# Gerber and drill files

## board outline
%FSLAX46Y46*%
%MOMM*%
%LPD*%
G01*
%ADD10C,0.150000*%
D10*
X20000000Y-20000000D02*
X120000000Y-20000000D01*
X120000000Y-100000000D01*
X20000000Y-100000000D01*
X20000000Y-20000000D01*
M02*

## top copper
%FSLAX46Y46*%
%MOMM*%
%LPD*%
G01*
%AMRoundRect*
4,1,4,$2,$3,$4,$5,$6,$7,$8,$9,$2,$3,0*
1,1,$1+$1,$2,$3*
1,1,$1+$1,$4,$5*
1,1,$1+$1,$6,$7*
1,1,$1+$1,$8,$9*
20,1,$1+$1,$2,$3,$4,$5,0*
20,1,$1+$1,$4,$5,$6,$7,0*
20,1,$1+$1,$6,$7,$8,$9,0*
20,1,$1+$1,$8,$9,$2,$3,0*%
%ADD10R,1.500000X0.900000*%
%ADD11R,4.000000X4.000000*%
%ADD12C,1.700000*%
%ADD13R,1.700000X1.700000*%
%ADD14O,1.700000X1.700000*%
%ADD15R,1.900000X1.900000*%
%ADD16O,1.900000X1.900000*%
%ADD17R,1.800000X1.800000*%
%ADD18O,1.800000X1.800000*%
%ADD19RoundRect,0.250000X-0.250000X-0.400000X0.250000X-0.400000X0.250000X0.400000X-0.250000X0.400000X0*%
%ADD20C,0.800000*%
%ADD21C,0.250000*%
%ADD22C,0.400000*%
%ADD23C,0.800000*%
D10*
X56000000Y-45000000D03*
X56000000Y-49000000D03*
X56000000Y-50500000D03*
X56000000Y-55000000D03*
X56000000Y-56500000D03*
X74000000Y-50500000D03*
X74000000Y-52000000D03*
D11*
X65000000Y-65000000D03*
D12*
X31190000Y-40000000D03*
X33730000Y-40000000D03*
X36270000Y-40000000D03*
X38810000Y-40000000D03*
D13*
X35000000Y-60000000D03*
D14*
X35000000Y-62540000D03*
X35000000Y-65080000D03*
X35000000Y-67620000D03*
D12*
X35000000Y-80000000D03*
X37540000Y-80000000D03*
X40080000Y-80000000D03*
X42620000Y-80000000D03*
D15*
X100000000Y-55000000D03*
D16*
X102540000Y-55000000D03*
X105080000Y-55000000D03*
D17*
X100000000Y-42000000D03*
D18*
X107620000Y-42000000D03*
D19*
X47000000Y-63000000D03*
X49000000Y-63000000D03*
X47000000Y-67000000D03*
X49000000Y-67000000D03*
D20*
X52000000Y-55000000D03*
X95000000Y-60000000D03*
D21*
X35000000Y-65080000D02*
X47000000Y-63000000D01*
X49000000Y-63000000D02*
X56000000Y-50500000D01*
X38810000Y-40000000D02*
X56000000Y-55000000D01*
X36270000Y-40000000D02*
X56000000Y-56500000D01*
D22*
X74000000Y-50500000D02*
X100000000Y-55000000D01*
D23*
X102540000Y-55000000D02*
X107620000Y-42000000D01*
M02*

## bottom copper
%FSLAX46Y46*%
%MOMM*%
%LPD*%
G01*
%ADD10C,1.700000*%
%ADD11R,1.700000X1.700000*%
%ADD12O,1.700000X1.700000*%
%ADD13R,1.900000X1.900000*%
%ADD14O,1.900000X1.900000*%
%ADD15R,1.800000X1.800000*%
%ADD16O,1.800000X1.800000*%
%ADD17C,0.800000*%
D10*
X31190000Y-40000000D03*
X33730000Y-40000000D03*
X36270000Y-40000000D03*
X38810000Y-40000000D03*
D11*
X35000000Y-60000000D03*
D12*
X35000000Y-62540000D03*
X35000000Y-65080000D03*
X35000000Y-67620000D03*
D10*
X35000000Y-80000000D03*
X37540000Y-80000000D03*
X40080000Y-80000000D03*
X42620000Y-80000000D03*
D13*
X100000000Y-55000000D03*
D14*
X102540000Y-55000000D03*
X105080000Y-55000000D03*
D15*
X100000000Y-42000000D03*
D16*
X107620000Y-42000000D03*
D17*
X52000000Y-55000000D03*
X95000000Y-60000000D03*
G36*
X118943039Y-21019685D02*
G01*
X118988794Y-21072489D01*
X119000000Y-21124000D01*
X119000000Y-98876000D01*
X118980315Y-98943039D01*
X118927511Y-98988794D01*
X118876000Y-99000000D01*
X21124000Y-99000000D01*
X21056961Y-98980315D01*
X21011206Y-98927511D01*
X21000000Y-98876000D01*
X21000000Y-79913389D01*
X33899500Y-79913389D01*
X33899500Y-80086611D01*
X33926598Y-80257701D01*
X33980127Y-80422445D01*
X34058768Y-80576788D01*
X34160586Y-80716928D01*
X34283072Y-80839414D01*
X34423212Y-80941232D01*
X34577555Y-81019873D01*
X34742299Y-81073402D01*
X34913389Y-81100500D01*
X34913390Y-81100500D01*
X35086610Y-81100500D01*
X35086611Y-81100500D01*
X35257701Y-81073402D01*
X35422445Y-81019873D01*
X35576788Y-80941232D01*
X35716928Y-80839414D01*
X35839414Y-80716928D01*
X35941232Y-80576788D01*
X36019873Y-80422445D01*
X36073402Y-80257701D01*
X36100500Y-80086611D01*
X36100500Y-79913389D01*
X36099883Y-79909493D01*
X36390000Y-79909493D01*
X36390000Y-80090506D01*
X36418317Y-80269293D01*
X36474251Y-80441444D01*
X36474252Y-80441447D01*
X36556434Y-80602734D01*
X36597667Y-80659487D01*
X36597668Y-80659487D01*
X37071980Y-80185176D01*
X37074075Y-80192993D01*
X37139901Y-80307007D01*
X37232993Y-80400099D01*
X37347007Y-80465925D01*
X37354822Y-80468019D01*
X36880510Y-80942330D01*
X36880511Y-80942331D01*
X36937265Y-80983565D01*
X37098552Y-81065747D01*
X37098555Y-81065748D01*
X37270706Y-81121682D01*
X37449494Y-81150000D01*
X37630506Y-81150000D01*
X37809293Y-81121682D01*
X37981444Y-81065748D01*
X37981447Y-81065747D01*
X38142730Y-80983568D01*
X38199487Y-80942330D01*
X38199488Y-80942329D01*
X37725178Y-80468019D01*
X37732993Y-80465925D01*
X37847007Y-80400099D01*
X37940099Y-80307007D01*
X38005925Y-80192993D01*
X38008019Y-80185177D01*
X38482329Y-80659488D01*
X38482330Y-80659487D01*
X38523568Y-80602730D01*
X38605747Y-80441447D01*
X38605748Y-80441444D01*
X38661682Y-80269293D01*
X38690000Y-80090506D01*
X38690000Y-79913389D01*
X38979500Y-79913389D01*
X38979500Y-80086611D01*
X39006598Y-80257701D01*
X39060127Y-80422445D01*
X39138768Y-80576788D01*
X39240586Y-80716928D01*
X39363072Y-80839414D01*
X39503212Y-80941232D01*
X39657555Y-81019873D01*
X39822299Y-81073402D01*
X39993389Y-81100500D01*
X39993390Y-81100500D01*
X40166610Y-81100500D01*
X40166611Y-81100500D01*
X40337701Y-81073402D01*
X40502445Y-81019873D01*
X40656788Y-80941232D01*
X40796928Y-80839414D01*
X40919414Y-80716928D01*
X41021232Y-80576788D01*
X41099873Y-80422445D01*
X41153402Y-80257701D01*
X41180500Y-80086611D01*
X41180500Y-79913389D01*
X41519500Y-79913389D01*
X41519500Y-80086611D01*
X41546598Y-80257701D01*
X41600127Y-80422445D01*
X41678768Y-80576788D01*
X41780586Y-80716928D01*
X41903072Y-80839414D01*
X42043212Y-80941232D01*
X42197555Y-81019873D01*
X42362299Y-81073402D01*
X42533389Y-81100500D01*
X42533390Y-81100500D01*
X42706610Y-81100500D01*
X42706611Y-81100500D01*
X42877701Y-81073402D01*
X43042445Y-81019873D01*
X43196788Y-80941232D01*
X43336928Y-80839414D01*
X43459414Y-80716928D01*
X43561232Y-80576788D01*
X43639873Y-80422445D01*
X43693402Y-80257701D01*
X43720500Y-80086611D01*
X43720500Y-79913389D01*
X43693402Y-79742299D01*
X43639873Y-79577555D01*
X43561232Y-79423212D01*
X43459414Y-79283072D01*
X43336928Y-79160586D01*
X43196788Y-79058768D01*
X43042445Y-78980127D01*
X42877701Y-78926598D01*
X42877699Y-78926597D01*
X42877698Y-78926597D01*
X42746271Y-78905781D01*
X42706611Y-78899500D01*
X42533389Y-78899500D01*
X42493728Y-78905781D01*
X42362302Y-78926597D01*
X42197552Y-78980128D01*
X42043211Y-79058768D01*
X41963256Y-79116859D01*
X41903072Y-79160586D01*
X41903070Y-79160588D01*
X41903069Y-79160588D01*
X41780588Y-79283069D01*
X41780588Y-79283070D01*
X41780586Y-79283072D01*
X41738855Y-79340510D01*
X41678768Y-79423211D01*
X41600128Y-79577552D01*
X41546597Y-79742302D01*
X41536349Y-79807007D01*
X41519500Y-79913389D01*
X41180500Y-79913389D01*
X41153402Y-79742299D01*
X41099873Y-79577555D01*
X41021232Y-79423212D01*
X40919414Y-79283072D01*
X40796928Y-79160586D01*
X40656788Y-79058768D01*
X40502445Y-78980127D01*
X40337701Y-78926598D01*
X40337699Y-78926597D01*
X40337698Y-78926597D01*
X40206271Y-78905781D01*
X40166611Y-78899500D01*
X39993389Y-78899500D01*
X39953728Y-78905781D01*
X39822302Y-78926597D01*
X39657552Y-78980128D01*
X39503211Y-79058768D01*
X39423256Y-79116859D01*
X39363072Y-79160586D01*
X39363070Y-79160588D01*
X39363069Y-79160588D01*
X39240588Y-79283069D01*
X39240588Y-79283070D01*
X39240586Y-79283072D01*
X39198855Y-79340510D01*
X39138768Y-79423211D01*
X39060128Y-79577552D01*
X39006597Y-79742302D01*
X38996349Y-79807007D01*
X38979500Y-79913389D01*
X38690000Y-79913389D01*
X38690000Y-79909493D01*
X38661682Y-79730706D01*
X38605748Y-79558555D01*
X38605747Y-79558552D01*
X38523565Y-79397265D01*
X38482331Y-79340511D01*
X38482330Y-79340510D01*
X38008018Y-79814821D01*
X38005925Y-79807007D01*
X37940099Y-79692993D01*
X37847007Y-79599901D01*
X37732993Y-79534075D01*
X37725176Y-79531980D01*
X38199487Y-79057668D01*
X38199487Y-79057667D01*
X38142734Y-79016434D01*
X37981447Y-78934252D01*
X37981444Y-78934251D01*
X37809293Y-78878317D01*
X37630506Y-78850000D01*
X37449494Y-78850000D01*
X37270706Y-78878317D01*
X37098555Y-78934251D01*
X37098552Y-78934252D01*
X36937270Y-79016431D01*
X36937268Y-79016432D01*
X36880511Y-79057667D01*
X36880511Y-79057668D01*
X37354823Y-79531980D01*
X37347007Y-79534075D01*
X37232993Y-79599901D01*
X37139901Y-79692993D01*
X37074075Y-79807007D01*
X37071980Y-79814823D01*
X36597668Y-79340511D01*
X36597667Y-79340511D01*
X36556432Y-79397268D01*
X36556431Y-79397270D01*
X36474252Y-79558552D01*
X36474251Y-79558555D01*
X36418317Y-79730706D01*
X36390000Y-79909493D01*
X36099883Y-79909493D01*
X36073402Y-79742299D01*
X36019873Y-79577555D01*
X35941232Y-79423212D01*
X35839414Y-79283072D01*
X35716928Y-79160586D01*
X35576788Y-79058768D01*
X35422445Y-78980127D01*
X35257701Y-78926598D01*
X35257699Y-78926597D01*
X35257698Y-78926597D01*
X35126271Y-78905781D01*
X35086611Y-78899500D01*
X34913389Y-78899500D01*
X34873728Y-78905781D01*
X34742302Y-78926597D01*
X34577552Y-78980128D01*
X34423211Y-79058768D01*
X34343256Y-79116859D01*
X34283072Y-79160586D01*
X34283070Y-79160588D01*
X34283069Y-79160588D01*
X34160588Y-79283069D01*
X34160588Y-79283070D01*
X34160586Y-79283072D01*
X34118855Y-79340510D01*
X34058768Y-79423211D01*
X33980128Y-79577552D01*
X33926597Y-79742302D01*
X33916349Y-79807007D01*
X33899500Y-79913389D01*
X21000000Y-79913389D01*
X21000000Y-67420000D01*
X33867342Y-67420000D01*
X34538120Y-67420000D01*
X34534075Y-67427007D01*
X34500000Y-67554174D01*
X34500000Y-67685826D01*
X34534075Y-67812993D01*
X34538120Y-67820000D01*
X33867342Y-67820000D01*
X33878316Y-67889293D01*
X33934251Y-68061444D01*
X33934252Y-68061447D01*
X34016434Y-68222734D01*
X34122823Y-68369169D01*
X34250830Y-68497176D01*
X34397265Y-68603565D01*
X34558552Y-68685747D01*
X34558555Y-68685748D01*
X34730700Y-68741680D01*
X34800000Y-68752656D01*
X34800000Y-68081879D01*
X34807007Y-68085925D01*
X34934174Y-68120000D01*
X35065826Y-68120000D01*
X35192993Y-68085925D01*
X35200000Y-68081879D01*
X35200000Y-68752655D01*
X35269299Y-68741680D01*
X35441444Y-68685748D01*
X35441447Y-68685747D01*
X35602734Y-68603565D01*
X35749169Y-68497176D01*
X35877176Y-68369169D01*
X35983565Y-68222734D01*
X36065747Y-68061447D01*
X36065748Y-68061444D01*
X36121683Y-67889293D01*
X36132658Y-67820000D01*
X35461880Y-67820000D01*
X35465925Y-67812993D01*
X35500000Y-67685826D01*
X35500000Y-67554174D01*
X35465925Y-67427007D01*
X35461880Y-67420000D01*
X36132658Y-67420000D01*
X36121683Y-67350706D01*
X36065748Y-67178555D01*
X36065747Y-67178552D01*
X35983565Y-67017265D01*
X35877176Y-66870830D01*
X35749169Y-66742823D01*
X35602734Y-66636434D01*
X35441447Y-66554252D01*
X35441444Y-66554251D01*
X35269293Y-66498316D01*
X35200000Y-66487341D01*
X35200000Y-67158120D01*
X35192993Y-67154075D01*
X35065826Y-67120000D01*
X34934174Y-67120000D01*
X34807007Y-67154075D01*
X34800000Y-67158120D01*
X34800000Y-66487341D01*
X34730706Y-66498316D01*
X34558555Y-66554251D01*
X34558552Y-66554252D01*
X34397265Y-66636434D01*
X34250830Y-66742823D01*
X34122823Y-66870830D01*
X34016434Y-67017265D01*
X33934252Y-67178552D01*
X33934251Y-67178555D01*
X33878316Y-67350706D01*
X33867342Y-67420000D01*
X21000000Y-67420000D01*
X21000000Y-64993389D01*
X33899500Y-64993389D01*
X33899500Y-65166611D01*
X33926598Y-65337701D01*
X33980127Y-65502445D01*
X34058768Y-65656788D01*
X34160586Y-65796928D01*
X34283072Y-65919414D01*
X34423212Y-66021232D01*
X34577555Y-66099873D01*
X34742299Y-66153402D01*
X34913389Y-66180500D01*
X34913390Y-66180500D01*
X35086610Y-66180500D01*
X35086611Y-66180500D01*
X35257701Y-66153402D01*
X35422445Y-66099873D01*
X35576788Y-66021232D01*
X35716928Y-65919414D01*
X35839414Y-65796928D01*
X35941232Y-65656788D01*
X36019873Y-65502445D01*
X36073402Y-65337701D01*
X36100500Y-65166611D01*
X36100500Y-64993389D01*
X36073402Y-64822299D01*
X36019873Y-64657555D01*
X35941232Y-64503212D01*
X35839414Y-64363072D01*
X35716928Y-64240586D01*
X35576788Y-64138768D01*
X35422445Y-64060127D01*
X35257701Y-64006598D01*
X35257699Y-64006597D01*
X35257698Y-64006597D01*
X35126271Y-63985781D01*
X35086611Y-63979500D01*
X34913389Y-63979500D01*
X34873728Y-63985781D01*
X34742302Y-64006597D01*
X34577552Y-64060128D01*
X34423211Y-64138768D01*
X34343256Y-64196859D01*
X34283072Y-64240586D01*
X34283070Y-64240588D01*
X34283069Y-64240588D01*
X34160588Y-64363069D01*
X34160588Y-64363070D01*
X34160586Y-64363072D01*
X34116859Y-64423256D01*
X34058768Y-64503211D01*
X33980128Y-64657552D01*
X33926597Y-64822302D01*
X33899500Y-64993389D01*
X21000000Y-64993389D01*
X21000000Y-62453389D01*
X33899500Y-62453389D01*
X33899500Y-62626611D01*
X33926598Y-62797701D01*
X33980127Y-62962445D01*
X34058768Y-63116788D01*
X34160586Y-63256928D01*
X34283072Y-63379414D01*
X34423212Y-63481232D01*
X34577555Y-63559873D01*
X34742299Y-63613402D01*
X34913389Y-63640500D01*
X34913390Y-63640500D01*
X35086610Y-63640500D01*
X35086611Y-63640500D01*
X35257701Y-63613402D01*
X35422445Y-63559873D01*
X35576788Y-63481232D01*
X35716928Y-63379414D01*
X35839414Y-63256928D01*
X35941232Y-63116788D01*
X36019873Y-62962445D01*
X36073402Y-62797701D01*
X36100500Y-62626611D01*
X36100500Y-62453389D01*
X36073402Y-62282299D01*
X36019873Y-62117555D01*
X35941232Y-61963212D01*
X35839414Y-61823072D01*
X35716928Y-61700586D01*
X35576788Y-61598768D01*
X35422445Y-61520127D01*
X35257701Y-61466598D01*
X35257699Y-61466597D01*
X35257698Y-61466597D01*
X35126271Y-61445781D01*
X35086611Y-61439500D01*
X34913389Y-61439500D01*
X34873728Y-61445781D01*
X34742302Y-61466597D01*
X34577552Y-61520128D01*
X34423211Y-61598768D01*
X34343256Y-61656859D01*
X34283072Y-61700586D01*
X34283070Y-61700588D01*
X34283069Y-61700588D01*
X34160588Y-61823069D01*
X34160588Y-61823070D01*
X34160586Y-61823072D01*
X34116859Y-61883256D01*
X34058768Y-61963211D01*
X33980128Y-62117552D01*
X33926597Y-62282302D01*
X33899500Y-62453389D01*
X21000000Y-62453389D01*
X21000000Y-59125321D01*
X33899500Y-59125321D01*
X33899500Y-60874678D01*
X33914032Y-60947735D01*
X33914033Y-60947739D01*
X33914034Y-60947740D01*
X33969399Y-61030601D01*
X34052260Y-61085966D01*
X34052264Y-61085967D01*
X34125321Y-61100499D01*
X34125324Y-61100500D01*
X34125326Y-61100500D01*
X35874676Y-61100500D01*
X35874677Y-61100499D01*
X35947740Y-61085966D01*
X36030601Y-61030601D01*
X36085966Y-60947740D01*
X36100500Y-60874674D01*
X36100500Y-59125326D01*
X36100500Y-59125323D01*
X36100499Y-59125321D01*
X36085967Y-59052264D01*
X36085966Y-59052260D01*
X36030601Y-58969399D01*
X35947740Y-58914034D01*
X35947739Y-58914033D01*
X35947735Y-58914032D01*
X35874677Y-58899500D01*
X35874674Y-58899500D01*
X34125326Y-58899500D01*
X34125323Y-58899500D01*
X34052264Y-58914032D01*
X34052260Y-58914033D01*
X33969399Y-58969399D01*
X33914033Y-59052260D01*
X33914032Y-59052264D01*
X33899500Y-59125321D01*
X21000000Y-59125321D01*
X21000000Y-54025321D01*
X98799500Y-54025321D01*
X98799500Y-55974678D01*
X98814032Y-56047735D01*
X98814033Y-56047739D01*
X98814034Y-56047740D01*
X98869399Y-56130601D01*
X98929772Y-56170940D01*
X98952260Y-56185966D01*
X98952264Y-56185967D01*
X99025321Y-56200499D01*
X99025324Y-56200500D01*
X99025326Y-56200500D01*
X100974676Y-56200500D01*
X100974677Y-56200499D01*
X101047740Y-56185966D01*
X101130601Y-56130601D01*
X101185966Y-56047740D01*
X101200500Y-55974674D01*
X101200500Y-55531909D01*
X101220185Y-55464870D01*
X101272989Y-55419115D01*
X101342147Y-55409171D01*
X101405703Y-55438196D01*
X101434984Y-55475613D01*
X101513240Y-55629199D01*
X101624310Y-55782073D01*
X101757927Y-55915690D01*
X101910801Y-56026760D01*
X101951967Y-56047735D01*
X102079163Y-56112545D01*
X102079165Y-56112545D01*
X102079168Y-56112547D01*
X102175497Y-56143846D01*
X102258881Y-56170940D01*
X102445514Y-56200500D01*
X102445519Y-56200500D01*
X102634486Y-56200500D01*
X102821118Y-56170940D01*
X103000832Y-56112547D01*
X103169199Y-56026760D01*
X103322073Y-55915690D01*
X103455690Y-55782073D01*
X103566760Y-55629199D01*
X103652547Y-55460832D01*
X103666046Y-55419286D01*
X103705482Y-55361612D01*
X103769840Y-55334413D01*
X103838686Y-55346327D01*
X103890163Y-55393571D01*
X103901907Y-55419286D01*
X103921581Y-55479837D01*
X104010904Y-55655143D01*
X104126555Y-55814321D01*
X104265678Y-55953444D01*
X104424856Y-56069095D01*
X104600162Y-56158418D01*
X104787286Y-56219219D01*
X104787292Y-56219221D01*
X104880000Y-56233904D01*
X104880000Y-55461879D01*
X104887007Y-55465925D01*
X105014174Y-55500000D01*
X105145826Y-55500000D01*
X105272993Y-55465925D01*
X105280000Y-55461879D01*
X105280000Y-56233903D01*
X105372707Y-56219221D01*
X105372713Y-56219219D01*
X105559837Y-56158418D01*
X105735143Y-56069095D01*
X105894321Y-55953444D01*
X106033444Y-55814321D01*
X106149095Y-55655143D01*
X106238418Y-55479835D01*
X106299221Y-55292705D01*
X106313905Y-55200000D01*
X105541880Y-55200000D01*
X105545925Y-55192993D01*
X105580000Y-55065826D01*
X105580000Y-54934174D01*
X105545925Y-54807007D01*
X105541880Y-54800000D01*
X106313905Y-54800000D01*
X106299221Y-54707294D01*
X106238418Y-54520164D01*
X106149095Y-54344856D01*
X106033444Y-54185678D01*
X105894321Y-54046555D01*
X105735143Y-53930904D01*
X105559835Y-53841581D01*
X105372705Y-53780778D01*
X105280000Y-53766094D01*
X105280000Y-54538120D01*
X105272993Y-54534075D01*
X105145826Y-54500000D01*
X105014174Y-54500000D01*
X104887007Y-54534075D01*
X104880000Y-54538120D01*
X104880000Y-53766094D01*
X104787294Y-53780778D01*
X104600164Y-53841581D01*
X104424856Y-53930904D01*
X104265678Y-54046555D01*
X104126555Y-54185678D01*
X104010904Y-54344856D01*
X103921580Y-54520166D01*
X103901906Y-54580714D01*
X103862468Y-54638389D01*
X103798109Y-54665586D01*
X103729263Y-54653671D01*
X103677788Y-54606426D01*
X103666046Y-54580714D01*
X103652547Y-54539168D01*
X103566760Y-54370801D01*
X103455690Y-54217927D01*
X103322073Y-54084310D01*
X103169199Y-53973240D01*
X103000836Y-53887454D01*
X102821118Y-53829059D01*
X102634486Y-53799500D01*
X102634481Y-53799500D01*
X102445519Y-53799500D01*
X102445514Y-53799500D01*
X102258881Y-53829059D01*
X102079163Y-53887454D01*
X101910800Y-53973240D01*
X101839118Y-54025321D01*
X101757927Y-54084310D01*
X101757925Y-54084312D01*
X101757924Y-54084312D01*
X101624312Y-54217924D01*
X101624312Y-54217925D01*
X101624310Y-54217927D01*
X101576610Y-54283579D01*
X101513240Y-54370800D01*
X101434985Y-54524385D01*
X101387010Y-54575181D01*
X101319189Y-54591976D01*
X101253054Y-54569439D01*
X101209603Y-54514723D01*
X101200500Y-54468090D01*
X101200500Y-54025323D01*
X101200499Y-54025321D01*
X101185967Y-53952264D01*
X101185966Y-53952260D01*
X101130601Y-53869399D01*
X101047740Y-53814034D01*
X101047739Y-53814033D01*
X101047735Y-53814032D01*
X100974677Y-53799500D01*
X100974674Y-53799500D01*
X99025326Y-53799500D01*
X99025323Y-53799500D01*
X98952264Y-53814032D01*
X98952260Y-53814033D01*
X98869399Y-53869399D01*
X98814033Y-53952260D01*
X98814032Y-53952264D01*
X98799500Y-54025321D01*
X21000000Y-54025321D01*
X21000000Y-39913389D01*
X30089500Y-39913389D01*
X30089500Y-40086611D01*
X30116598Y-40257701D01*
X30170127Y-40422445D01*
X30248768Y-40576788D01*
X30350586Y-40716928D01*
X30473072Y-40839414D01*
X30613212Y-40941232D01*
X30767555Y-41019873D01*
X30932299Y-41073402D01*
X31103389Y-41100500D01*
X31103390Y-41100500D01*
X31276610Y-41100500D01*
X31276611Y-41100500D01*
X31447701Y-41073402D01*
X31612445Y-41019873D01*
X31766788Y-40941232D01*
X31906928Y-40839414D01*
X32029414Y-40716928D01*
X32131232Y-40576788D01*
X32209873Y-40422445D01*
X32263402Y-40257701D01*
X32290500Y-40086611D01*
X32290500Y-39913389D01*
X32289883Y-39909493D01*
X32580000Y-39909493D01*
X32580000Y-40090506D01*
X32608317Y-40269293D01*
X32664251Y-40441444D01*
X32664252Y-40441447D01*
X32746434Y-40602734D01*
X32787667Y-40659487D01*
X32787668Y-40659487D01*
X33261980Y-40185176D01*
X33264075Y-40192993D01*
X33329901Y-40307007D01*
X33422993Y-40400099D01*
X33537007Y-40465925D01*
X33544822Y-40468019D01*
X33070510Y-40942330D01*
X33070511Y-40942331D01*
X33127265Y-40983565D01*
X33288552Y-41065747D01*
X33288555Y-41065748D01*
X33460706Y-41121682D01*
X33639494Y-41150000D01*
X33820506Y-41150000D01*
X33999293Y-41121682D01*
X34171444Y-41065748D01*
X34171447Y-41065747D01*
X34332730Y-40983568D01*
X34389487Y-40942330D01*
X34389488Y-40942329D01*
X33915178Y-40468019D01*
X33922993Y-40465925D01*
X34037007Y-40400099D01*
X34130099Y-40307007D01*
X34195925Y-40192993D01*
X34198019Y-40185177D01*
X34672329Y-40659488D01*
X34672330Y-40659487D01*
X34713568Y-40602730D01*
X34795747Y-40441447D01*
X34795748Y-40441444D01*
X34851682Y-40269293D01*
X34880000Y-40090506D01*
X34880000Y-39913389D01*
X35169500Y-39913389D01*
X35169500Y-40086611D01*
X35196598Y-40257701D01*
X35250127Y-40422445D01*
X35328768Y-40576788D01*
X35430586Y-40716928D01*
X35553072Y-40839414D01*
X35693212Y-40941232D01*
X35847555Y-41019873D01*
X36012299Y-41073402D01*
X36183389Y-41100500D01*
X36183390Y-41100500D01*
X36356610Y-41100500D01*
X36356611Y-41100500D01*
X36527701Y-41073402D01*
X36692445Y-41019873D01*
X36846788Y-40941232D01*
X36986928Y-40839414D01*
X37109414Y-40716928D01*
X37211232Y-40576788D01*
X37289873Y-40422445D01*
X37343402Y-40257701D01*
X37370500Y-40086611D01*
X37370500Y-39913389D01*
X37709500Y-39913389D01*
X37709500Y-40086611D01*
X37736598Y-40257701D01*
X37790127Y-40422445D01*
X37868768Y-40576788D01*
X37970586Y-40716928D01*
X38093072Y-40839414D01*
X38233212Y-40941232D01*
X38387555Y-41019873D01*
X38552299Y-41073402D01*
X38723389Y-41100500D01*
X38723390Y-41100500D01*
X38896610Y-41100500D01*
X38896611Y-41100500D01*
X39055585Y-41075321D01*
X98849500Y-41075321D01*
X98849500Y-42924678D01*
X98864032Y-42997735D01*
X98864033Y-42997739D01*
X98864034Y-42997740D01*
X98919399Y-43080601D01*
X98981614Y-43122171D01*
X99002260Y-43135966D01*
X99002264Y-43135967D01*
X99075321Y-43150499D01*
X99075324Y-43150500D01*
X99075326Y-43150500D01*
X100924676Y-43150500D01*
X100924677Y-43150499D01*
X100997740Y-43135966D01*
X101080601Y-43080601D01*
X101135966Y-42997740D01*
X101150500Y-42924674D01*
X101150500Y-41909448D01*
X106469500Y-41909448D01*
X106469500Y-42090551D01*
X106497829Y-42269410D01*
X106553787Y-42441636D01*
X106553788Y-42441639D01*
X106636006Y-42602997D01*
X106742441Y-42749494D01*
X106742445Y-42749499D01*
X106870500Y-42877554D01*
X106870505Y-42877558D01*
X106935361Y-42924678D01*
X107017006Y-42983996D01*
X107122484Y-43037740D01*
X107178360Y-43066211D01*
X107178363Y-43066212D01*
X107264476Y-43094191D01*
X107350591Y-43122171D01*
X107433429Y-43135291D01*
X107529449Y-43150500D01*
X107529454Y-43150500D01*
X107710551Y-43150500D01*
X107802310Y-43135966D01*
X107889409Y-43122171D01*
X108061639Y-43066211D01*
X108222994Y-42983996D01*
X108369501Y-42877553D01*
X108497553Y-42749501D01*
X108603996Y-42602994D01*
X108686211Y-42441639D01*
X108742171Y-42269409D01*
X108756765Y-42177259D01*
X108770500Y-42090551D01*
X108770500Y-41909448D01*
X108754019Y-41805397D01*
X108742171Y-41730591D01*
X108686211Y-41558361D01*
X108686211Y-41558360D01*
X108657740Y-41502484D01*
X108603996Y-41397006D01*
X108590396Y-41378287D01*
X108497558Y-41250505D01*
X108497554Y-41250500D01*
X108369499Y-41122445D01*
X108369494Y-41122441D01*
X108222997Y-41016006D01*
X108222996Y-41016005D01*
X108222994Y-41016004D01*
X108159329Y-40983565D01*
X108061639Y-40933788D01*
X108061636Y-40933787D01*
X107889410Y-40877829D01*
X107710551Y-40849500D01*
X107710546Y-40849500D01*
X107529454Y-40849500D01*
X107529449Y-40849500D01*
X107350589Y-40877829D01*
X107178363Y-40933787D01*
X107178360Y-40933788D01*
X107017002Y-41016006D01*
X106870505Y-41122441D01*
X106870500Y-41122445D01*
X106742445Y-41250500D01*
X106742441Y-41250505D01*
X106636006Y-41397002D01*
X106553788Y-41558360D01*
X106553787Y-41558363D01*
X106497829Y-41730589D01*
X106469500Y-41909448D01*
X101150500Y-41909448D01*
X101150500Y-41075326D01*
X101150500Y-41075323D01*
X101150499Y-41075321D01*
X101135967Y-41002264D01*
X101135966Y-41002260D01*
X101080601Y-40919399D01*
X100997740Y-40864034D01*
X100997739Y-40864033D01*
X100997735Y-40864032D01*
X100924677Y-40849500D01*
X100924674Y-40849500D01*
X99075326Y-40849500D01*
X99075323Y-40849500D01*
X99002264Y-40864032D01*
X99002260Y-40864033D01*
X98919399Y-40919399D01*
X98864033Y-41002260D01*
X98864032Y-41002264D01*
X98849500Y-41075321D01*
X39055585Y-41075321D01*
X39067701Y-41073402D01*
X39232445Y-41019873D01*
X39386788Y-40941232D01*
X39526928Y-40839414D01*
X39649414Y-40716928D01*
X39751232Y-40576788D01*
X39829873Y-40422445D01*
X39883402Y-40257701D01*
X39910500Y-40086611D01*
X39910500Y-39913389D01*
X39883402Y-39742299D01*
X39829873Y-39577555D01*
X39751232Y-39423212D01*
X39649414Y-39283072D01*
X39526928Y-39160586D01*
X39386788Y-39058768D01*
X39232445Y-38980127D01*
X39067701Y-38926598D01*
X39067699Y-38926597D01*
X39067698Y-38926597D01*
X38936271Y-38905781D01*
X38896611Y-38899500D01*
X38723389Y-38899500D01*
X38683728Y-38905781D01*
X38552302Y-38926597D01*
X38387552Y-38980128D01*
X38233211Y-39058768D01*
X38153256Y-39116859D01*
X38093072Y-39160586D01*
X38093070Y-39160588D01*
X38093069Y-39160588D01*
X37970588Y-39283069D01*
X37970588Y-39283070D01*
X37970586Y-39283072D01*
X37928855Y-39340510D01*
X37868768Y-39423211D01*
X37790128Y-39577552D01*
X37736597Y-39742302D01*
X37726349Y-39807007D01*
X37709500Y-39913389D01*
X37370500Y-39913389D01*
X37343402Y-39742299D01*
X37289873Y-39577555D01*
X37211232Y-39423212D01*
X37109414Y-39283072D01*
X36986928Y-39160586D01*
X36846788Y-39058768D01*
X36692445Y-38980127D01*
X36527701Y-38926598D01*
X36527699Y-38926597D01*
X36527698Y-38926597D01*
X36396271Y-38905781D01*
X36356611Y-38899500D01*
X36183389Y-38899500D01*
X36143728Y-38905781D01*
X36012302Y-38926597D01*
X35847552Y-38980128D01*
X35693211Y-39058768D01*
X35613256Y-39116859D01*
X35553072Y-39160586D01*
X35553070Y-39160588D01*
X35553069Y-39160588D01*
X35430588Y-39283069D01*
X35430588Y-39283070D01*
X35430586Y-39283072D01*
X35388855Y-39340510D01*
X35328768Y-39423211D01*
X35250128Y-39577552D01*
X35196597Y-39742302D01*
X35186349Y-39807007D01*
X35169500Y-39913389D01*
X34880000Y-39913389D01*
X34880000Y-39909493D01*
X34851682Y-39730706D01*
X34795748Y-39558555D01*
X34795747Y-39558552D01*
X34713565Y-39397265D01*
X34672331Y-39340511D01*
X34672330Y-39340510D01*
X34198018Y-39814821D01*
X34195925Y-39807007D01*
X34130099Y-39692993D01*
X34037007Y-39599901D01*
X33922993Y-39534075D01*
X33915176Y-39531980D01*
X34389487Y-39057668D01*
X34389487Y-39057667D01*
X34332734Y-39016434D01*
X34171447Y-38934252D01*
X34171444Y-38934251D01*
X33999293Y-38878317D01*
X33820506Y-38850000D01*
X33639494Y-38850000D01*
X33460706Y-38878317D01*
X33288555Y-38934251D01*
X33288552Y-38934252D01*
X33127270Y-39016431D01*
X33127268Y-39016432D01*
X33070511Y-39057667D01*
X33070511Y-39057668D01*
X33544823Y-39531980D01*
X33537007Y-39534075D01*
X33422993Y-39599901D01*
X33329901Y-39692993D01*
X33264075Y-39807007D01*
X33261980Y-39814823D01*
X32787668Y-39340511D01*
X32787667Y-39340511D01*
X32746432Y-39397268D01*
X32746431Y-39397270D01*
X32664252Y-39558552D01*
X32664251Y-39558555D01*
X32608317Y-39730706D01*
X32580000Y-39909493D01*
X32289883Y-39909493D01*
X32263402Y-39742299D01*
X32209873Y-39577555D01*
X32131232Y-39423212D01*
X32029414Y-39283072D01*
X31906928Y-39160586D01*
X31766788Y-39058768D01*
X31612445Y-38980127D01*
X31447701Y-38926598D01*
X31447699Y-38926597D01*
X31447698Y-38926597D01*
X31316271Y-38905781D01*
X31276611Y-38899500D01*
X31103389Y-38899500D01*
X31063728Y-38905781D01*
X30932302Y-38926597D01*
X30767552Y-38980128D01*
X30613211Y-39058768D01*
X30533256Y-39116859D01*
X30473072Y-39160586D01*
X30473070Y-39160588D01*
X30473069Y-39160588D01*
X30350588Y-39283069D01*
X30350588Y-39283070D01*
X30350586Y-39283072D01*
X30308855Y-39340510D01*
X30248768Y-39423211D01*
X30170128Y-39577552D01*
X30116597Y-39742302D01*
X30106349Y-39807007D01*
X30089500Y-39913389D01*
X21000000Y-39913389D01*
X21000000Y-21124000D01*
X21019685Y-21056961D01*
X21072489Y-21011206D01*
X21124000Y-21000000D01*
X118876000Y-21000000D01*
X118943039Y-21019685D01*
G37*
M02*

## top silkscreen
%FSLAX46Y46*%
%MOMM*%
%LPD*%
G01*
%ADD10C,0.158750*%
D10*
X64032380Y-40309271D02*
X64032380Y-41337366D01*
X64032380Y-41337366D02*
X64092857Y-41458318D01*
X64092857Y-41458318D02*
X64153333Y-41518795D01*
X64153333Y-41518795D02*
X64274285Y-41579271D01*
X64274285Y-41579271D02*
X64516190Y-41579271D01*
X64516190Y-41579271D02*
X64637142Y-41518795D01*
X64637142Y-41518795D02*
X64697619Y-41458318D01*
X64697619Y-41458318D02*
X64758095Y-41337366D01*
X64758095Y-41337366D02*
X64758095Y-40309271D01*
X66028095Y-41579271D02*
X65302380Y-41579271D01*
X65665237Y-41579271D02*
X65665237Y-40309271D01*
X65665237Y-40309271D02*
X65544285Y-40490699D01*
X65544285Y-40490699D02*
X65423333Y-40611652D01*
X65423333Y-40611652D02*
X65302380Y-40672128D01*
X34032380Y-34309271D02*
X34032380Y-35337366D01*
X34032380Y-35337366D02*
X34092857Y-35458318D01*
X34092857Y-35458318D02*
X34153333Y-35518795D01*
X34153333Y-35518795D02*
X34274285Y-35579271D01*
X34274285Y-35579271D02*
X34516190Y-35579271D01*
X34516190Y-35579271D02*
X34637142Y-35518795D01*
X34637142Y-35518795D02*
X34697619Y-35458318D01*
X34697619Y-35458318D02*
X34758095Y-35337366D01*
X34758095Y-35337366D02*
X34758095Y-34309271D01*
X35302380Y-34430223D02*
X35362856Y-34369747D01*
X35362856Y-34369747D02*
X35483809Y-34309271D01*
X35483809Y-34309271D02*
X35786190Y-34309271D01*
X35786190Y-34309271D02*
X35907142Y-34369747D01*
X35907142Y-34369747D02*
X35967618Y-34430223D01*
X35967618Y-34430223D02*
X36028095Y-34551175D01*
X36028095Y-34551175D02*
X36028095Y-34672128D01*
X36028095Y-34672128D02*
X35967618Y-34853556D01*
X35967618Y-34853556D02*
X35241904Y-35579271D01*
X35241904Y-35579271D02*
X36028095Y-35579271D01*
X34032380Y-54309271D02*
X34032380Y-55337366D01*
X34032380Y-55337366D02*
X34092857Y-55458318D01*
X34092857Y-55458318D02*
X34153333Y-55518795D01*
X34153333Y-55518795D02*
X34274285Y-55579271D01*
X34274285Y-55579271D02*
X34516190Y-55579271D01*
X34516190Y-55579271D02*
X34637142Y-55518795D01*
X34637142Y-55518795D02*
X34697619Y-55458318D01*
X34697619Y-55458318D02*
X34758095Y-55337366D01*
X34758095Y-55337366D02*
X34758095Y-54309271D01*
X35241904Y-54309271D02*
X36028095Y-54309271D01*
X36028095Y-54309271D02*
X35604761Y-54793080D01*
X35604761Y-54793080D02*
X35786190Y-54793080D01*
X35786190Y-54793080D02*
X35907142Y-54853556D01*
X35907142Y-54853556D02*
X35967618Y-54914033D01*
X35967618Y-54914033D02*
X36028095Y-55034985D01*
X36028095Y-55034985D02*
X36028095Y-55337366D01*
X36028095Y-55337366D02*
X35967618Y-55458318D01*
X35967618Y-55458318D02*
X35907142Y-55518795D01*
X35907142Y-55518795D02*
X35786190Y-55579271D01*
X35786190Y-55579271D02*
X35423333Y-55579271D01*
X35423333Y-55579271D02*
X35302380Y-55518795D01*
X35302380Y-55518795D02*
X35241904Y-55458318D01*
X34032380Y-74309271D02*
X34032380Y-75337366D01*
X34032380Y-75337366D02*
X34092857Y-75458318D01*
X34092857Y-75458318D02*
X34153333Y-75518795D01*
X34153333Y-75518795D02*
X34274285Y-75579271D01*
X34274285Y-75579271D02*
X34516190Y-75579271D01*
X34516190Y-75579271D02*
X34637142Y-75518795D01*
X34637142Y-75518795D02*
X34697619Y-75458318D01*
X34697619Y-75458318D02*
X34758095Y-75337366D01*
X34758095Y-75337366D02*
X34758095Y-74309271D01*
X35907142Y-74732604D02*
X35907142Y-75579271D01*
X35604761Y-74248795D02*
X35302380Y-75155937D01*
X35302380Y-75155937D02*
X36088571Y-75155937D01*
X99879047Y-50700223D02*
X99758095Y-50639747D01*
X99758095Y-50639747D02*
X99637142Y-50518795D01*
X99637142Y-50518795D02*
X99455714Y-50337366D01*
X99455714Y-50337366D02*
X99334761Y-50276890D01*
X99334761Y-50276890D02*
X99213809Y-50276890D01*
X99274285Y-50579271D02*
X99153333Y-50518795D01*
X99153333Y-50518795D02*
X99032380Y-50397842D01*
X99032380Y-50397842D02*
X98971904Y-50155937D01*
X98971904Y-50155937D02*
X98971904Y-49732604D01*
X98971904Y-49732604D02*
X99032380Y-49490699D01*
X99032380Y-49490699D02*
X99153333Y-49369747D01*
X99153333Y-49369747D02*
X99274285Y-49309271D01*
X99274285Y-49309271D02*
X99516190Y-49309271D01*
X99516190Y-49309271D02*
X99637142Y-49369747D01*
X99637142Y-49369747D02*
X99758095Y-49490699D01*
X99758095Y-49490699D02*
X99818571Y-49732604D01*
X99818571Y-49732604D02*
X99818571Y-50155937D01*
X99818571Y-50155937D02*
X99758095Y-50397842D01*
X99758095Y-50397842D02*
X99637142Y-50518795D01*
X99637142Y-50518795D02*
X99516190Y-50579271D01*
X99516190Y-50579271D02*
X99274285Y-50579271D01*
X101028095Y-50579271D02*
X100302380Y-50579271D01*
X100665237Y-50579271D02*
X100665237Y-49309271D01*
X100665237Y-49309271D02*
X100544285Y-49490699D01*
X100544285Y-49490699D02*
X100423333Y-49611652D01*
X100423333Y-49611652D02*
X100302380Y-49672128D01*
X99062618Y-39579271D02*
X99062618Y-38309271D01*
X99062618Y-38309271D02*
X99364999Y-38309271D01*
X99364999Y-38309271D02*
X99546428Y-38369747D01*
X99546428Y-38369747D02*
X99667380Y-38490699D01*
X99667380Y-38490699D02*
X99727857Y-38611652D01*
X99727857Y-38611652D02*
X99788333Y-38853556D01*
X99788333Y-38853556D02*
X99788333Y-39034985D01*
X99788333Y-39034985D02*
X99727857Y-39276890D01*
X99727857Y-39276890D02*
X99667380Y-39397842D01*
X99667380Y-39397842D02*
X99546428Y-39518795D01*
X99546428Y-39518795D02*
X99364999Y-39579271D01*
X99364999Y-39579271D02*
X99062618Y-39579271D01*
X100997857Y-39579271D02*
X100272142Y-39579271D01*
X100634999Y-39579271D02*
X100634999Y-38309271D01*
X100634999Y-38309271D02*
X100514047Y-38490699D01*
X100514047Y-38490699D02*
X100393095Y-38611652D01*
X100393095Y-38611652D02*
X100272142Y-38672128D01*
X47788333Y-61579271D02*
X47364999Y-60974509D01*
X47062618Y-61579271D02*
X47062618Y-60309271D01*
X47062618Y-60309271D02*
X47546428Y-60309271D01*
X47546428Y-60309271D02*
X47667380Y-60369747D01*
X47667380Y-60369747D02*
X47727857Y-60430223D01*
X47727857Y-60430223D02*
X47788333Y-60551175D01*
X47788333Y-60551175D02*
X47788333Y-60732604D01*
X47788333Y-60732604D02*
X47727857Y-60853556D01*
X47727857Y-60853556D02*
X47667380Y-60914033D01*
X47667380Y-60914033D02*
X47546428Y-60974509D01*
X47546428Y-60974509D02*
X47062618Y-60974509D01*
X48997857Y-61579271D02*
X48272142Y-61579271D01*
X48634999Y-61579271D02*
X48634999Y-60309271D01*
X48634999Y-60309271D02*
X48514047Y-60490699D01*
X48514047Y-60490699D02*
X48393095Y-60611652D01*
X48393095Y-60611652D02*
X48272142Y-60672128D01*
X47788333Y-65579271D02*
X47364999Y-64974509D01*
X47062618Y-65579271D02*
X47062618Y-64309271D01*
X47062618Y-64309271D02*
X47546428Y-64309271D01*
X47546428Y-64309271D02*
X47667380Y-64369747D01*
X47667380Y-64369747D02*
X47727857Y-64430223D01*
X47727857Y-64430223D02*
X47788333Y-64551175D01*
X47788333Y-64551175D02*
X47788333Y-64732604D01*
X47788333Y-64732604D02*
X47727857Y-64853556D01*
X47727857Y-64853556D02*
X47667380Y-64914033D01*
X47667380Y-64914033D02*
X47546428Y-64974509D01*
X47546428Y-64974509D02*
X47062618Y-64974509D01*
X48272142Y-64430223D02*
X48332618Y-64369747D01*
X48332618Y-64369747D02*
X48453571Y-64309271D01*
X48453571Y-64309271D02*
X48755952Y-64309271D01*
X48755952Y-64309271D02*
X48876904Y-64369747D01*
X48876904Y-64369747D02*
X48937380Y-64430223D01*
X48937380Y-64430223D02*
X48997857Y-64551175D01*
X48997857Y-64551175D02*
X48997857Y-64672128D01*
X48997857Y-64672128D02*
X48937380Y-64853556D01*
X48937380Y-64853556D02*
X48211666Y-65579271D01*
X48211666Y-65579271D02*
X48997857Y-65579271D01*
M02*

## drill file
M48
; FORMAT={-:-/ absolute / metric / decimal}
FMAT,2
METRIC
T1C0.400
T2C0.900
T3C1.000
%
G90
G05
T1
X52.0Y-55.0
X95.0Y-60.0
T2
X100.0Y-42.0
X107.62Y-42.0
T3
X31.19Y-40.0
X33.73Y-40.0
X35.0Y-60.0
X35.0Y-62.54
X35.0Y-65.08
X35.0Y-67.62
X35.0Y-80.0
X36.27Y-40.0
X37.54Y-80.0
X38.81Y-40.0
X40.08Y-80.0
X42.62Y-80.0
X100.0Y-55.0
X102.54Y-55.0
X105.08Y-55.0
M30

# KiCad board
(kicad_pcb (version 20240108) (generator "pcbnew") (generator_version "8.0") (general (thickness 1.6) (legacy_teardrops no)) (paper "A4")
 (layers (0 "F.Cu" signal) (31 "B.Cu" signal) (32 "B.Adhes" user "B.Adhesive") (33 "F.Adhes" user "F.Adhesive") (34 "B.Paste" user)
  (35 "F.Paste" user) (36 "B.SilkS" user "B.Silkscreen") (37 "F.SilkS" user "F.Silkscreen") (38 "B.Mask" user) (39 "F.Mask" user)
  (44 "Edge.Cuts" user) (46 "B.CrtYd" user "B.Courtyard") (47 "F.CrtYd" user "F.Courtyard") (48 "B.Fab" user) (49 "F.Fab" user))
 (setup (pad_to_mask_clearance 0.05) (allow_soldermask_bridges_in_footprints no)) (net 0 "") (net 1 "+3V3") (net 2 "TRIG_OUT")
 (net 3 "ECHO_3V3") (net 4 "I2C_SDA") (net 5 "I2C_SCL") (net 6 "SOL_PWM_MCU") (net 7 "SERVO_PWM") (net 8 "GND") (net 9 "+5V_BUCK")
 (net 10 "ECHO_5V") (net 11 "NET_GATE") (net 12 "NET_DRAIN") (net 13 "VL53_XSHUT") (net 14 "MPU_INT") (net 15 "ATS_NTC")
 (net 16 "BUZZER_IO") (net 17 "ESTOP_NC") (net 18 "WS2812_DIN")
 (gr_rect (start 20 20) (end 120 100) (stroke (width 0.15) (type default)) (fill none) (layer "Edge.Cuts"))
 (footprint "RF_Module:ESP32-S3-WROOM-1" (layer "F.Cu") (at 65 55) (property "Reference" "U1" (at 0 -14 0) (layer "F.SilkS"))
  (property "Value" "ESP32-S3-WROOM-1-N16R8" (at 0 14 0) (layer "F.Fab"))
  (pad "1" smd rect (at -9.0 -10.0) (size 1.5 0.9) (layers "F.Cu" "F.Paste" "F.Mask") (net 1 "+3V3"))
  (pad "4" smd rect (at -9.0 -6.0) (size 1.5 0.9) (layers "F.Cu" "F.Paste" "F.Mask") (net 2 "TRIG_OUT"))
  (pad "5" smd rect (at -9.0 -4.5) (size 1.5 0.9) (layers "F.Cu" "F.Paste" "F.Mask") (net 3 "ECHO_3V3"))
  (pad "8" smd rect (at -9.0 0.0) (size 1.5 0.9) (layers "F.Cu" "F.Paste" "F.Mask") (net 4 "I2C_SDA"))
  (pad "9" smd rect (at -9.0 1.5) (size 1.5 0.9) (layers "F.Cu" "F.Paste" "F.Mask") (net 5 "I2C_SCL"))
  (pad "14" smd rect (at 9.0 -4.5) (size 1.5 0.9) (layers "F.Cu" "F.Paste" "F.Mask") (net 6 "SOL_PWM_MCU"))
  (pad "15" smd rect (at 9.0 -3.0) (size 1.5 0.9) (layers "F.Cu" "F.Paste" "F.Mask") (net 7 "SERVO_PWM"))
  (pad "40" smd rect (at 0.0 10.0) (size 4.0 4.0) (layers "F.Cu" "F.Paste" "F.Mask") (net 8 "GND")))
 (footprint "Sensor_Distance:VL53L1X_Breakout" (layer "F.Cu") (at 35 40) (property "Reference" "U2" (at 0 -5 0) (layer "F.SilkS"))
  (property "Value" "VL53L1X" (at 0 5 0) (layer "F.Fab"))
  (pad "1" thru_hole circle (at -3.81 0) (size 1.7 1.7) (drill 1.0) (layers "*.Cu" "*.Mask") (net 1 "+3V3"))
  (pad "2" thru_hole circle (at -1.27 0) (size 1.7 1.7) (drill 1.0) (layers "*.Cu" "*.Mask") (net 8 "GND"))
  (pad "3" thru_hole circle (at 1.27 0) (size 1.7 1.7) (drill 1.0) (layers "*.Cu" "*.Mask") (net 5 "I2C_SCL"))
  (pad "4" thru_hole circle (at 3.81 0) (size 1.7 1.7) (drill 1.0) (layers "*.Cu" "*.Mask") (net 4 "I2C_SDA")))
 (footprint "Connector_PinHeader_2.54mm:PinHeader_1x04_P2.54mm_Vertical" (layer "F.Cu") (at 35 60)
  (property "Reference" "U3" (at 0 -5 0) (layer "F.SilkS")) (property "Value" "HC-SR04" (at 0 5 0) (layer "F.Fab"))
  (pad "1" thru_hole rect (at 0 0) (size 1.7 1.7) (drill 1.0) (layers "*.Cu" "*.Mask") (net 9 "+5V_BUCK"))
  (pad "2" thru_hole oval (at 0 2.54) (size 1.7 1.7) (drill 1.0) (layers "*.Cu" "*.Mask") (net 2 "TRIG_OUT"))
  (pad "3" thru_hole oval (at 0 5.08) (size 1.7 1.7) (drill 1.0) (layers "*.Cu" "*.Mask") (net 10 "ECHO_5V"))
  (pad "4" thru_hole oval (at 0 7.62) (size 1.7 1.7) (drill 1.0) (layers "*.Cu" "*.Mask") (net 8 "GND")))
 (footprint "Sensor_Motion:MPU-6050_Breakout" (layer "F.Cu") (at 35 80) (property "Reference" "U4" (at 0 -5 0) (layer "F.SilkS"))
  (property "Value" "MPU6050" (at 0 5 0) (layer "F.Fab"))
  (pad "1" thru_hole circle (at 0 0) (size 1.7 1.7) (drill 1.0) (layers "*.Cu" "*.Mask") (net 1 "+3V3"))
  (pad "2" thru_hole circle (at 2.54 0) (size 1.7 1.7) (drill 1.0) (layers "*.Cu" "*.Mask") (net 8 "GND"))
  (pad "3" thru_hole circle (at 5.08 0) (size 1.7 1.7) (drill 1.0) (layers "*.Cu" "*.Mask") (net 5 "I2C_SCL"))
  (pad "4" thru_hole circle (at 7.62 0) (size 1.7 1.7) (drill 1.0) (layers "*.Cu" "*.Mask") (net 4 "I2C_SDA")))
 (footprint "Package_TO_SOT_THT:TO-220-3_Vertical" (layer "F.Cu") (at 100 55) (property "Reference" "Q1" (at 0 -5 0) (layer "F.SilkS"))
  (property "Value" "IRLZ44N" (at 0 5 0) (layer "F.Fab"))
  (pad "1" thru_hole rect (at 0 0) (size 1.9 1.9) (drill 1.0) (layers "*.Cu" "*.Mask") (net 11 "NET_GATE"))
  (pad "2" thru_hole oval (at 2.54 0) (size 1.9 1.9) (drill 1.0) (layers "*.Cu" "*.Mask") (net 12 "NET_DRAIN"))
  (pad "3" thru_hole oval (at 5.08 0) (size 1.9 1.9) (drill 1.0) (layers "*.Cu" "*.Mask") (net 8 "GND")))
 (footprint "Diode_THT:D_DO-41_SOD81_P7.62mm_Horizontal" (layer "F.Cu") (at 100 42)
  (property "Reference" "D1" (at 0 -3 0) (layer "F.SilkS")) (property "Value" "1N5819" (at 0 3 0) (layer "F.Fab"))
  (pad "1" thru_hole rect (at 0 0) (size 1.8 1.8) (drill 0.9) (layers "*.Cu" "*.Mask") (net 9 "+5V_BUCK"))
  (pad "2" thru_hole oval (at 7.62 0) (size 1.8 1.8) (drill 0.9) (layers "*.Cu" "*.Mask") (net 12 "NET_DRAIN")))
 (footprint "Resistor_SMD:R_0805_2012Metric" (layer "F.Cu") (at 48 63) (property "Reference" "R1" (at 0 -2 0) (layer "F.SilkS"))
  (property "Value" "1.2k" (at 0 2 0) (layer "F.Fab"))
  (pad "1" smd roundrect (at -1.0 0) (size 1.0 1.3) (layers "F.Cu" "F.Paste" "F.Mask") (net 10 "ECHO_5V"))
  (pad "2" smd roundrect (at 1.0 0) (size 1.0 1.3) (layers "F.Cu" "F.Paste" "F.Mask") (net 3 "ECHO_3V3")))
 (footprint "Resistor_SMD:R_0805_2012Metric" (layer "F.Cu") (at 48 67) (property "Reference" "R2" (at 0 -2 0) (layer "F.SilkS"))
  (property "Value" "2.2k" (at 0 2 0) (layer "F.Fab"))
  (pad "1" smd roundrect (at -1.0 0) (size 1.0 1.3) (layers "F.Cu" "F.Paste" "F.Mask") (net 3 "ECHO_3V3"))
  (pad "2" smd roundrect (at 1.0 0) (size 1.0 1.3) (layers "F.Cu" "F.Paste" "F.Mask") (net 8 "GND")))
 (segment (start 35 65.08) (end 47 63.0) (width 0.25) (layer "F.Cu") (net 10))
 (segment (start 49 63.0) (end 56 50.5) (width 0.25) (layer "F.Cu") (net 3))
 (segment (start 38.81 40.0) (end 56 55.0) (width 0.25) (layer "F.Cu") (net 4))
 (segment (start 36.27 40.0) (end 56 56.5) (width 0.25) (layer "F.Cu") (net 5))
 (segment (start 74 50.5) (end 100 55.0) (width 0.4) (layer "F.Cu") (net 11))
 (segment (start 102.54 55.0) (end 107.62 42.0) (width 0.8) (layer "F.Cu") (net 12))
 (via (at 52 55) (size 0.8) (drill 0.4) (layers "F.Cu" "B.Cu") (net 8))
 (via (at 95 60) (size 0.8) (drill 0.4) (layers "F.Cu" "B.Cu") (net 8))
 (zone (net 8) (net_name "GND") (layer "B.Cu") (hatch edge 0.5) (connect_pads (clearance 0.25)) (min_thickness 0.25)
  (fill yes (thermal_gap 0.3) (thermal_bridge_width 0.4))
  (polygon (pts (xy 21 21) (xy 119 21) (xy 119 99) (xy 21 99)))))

